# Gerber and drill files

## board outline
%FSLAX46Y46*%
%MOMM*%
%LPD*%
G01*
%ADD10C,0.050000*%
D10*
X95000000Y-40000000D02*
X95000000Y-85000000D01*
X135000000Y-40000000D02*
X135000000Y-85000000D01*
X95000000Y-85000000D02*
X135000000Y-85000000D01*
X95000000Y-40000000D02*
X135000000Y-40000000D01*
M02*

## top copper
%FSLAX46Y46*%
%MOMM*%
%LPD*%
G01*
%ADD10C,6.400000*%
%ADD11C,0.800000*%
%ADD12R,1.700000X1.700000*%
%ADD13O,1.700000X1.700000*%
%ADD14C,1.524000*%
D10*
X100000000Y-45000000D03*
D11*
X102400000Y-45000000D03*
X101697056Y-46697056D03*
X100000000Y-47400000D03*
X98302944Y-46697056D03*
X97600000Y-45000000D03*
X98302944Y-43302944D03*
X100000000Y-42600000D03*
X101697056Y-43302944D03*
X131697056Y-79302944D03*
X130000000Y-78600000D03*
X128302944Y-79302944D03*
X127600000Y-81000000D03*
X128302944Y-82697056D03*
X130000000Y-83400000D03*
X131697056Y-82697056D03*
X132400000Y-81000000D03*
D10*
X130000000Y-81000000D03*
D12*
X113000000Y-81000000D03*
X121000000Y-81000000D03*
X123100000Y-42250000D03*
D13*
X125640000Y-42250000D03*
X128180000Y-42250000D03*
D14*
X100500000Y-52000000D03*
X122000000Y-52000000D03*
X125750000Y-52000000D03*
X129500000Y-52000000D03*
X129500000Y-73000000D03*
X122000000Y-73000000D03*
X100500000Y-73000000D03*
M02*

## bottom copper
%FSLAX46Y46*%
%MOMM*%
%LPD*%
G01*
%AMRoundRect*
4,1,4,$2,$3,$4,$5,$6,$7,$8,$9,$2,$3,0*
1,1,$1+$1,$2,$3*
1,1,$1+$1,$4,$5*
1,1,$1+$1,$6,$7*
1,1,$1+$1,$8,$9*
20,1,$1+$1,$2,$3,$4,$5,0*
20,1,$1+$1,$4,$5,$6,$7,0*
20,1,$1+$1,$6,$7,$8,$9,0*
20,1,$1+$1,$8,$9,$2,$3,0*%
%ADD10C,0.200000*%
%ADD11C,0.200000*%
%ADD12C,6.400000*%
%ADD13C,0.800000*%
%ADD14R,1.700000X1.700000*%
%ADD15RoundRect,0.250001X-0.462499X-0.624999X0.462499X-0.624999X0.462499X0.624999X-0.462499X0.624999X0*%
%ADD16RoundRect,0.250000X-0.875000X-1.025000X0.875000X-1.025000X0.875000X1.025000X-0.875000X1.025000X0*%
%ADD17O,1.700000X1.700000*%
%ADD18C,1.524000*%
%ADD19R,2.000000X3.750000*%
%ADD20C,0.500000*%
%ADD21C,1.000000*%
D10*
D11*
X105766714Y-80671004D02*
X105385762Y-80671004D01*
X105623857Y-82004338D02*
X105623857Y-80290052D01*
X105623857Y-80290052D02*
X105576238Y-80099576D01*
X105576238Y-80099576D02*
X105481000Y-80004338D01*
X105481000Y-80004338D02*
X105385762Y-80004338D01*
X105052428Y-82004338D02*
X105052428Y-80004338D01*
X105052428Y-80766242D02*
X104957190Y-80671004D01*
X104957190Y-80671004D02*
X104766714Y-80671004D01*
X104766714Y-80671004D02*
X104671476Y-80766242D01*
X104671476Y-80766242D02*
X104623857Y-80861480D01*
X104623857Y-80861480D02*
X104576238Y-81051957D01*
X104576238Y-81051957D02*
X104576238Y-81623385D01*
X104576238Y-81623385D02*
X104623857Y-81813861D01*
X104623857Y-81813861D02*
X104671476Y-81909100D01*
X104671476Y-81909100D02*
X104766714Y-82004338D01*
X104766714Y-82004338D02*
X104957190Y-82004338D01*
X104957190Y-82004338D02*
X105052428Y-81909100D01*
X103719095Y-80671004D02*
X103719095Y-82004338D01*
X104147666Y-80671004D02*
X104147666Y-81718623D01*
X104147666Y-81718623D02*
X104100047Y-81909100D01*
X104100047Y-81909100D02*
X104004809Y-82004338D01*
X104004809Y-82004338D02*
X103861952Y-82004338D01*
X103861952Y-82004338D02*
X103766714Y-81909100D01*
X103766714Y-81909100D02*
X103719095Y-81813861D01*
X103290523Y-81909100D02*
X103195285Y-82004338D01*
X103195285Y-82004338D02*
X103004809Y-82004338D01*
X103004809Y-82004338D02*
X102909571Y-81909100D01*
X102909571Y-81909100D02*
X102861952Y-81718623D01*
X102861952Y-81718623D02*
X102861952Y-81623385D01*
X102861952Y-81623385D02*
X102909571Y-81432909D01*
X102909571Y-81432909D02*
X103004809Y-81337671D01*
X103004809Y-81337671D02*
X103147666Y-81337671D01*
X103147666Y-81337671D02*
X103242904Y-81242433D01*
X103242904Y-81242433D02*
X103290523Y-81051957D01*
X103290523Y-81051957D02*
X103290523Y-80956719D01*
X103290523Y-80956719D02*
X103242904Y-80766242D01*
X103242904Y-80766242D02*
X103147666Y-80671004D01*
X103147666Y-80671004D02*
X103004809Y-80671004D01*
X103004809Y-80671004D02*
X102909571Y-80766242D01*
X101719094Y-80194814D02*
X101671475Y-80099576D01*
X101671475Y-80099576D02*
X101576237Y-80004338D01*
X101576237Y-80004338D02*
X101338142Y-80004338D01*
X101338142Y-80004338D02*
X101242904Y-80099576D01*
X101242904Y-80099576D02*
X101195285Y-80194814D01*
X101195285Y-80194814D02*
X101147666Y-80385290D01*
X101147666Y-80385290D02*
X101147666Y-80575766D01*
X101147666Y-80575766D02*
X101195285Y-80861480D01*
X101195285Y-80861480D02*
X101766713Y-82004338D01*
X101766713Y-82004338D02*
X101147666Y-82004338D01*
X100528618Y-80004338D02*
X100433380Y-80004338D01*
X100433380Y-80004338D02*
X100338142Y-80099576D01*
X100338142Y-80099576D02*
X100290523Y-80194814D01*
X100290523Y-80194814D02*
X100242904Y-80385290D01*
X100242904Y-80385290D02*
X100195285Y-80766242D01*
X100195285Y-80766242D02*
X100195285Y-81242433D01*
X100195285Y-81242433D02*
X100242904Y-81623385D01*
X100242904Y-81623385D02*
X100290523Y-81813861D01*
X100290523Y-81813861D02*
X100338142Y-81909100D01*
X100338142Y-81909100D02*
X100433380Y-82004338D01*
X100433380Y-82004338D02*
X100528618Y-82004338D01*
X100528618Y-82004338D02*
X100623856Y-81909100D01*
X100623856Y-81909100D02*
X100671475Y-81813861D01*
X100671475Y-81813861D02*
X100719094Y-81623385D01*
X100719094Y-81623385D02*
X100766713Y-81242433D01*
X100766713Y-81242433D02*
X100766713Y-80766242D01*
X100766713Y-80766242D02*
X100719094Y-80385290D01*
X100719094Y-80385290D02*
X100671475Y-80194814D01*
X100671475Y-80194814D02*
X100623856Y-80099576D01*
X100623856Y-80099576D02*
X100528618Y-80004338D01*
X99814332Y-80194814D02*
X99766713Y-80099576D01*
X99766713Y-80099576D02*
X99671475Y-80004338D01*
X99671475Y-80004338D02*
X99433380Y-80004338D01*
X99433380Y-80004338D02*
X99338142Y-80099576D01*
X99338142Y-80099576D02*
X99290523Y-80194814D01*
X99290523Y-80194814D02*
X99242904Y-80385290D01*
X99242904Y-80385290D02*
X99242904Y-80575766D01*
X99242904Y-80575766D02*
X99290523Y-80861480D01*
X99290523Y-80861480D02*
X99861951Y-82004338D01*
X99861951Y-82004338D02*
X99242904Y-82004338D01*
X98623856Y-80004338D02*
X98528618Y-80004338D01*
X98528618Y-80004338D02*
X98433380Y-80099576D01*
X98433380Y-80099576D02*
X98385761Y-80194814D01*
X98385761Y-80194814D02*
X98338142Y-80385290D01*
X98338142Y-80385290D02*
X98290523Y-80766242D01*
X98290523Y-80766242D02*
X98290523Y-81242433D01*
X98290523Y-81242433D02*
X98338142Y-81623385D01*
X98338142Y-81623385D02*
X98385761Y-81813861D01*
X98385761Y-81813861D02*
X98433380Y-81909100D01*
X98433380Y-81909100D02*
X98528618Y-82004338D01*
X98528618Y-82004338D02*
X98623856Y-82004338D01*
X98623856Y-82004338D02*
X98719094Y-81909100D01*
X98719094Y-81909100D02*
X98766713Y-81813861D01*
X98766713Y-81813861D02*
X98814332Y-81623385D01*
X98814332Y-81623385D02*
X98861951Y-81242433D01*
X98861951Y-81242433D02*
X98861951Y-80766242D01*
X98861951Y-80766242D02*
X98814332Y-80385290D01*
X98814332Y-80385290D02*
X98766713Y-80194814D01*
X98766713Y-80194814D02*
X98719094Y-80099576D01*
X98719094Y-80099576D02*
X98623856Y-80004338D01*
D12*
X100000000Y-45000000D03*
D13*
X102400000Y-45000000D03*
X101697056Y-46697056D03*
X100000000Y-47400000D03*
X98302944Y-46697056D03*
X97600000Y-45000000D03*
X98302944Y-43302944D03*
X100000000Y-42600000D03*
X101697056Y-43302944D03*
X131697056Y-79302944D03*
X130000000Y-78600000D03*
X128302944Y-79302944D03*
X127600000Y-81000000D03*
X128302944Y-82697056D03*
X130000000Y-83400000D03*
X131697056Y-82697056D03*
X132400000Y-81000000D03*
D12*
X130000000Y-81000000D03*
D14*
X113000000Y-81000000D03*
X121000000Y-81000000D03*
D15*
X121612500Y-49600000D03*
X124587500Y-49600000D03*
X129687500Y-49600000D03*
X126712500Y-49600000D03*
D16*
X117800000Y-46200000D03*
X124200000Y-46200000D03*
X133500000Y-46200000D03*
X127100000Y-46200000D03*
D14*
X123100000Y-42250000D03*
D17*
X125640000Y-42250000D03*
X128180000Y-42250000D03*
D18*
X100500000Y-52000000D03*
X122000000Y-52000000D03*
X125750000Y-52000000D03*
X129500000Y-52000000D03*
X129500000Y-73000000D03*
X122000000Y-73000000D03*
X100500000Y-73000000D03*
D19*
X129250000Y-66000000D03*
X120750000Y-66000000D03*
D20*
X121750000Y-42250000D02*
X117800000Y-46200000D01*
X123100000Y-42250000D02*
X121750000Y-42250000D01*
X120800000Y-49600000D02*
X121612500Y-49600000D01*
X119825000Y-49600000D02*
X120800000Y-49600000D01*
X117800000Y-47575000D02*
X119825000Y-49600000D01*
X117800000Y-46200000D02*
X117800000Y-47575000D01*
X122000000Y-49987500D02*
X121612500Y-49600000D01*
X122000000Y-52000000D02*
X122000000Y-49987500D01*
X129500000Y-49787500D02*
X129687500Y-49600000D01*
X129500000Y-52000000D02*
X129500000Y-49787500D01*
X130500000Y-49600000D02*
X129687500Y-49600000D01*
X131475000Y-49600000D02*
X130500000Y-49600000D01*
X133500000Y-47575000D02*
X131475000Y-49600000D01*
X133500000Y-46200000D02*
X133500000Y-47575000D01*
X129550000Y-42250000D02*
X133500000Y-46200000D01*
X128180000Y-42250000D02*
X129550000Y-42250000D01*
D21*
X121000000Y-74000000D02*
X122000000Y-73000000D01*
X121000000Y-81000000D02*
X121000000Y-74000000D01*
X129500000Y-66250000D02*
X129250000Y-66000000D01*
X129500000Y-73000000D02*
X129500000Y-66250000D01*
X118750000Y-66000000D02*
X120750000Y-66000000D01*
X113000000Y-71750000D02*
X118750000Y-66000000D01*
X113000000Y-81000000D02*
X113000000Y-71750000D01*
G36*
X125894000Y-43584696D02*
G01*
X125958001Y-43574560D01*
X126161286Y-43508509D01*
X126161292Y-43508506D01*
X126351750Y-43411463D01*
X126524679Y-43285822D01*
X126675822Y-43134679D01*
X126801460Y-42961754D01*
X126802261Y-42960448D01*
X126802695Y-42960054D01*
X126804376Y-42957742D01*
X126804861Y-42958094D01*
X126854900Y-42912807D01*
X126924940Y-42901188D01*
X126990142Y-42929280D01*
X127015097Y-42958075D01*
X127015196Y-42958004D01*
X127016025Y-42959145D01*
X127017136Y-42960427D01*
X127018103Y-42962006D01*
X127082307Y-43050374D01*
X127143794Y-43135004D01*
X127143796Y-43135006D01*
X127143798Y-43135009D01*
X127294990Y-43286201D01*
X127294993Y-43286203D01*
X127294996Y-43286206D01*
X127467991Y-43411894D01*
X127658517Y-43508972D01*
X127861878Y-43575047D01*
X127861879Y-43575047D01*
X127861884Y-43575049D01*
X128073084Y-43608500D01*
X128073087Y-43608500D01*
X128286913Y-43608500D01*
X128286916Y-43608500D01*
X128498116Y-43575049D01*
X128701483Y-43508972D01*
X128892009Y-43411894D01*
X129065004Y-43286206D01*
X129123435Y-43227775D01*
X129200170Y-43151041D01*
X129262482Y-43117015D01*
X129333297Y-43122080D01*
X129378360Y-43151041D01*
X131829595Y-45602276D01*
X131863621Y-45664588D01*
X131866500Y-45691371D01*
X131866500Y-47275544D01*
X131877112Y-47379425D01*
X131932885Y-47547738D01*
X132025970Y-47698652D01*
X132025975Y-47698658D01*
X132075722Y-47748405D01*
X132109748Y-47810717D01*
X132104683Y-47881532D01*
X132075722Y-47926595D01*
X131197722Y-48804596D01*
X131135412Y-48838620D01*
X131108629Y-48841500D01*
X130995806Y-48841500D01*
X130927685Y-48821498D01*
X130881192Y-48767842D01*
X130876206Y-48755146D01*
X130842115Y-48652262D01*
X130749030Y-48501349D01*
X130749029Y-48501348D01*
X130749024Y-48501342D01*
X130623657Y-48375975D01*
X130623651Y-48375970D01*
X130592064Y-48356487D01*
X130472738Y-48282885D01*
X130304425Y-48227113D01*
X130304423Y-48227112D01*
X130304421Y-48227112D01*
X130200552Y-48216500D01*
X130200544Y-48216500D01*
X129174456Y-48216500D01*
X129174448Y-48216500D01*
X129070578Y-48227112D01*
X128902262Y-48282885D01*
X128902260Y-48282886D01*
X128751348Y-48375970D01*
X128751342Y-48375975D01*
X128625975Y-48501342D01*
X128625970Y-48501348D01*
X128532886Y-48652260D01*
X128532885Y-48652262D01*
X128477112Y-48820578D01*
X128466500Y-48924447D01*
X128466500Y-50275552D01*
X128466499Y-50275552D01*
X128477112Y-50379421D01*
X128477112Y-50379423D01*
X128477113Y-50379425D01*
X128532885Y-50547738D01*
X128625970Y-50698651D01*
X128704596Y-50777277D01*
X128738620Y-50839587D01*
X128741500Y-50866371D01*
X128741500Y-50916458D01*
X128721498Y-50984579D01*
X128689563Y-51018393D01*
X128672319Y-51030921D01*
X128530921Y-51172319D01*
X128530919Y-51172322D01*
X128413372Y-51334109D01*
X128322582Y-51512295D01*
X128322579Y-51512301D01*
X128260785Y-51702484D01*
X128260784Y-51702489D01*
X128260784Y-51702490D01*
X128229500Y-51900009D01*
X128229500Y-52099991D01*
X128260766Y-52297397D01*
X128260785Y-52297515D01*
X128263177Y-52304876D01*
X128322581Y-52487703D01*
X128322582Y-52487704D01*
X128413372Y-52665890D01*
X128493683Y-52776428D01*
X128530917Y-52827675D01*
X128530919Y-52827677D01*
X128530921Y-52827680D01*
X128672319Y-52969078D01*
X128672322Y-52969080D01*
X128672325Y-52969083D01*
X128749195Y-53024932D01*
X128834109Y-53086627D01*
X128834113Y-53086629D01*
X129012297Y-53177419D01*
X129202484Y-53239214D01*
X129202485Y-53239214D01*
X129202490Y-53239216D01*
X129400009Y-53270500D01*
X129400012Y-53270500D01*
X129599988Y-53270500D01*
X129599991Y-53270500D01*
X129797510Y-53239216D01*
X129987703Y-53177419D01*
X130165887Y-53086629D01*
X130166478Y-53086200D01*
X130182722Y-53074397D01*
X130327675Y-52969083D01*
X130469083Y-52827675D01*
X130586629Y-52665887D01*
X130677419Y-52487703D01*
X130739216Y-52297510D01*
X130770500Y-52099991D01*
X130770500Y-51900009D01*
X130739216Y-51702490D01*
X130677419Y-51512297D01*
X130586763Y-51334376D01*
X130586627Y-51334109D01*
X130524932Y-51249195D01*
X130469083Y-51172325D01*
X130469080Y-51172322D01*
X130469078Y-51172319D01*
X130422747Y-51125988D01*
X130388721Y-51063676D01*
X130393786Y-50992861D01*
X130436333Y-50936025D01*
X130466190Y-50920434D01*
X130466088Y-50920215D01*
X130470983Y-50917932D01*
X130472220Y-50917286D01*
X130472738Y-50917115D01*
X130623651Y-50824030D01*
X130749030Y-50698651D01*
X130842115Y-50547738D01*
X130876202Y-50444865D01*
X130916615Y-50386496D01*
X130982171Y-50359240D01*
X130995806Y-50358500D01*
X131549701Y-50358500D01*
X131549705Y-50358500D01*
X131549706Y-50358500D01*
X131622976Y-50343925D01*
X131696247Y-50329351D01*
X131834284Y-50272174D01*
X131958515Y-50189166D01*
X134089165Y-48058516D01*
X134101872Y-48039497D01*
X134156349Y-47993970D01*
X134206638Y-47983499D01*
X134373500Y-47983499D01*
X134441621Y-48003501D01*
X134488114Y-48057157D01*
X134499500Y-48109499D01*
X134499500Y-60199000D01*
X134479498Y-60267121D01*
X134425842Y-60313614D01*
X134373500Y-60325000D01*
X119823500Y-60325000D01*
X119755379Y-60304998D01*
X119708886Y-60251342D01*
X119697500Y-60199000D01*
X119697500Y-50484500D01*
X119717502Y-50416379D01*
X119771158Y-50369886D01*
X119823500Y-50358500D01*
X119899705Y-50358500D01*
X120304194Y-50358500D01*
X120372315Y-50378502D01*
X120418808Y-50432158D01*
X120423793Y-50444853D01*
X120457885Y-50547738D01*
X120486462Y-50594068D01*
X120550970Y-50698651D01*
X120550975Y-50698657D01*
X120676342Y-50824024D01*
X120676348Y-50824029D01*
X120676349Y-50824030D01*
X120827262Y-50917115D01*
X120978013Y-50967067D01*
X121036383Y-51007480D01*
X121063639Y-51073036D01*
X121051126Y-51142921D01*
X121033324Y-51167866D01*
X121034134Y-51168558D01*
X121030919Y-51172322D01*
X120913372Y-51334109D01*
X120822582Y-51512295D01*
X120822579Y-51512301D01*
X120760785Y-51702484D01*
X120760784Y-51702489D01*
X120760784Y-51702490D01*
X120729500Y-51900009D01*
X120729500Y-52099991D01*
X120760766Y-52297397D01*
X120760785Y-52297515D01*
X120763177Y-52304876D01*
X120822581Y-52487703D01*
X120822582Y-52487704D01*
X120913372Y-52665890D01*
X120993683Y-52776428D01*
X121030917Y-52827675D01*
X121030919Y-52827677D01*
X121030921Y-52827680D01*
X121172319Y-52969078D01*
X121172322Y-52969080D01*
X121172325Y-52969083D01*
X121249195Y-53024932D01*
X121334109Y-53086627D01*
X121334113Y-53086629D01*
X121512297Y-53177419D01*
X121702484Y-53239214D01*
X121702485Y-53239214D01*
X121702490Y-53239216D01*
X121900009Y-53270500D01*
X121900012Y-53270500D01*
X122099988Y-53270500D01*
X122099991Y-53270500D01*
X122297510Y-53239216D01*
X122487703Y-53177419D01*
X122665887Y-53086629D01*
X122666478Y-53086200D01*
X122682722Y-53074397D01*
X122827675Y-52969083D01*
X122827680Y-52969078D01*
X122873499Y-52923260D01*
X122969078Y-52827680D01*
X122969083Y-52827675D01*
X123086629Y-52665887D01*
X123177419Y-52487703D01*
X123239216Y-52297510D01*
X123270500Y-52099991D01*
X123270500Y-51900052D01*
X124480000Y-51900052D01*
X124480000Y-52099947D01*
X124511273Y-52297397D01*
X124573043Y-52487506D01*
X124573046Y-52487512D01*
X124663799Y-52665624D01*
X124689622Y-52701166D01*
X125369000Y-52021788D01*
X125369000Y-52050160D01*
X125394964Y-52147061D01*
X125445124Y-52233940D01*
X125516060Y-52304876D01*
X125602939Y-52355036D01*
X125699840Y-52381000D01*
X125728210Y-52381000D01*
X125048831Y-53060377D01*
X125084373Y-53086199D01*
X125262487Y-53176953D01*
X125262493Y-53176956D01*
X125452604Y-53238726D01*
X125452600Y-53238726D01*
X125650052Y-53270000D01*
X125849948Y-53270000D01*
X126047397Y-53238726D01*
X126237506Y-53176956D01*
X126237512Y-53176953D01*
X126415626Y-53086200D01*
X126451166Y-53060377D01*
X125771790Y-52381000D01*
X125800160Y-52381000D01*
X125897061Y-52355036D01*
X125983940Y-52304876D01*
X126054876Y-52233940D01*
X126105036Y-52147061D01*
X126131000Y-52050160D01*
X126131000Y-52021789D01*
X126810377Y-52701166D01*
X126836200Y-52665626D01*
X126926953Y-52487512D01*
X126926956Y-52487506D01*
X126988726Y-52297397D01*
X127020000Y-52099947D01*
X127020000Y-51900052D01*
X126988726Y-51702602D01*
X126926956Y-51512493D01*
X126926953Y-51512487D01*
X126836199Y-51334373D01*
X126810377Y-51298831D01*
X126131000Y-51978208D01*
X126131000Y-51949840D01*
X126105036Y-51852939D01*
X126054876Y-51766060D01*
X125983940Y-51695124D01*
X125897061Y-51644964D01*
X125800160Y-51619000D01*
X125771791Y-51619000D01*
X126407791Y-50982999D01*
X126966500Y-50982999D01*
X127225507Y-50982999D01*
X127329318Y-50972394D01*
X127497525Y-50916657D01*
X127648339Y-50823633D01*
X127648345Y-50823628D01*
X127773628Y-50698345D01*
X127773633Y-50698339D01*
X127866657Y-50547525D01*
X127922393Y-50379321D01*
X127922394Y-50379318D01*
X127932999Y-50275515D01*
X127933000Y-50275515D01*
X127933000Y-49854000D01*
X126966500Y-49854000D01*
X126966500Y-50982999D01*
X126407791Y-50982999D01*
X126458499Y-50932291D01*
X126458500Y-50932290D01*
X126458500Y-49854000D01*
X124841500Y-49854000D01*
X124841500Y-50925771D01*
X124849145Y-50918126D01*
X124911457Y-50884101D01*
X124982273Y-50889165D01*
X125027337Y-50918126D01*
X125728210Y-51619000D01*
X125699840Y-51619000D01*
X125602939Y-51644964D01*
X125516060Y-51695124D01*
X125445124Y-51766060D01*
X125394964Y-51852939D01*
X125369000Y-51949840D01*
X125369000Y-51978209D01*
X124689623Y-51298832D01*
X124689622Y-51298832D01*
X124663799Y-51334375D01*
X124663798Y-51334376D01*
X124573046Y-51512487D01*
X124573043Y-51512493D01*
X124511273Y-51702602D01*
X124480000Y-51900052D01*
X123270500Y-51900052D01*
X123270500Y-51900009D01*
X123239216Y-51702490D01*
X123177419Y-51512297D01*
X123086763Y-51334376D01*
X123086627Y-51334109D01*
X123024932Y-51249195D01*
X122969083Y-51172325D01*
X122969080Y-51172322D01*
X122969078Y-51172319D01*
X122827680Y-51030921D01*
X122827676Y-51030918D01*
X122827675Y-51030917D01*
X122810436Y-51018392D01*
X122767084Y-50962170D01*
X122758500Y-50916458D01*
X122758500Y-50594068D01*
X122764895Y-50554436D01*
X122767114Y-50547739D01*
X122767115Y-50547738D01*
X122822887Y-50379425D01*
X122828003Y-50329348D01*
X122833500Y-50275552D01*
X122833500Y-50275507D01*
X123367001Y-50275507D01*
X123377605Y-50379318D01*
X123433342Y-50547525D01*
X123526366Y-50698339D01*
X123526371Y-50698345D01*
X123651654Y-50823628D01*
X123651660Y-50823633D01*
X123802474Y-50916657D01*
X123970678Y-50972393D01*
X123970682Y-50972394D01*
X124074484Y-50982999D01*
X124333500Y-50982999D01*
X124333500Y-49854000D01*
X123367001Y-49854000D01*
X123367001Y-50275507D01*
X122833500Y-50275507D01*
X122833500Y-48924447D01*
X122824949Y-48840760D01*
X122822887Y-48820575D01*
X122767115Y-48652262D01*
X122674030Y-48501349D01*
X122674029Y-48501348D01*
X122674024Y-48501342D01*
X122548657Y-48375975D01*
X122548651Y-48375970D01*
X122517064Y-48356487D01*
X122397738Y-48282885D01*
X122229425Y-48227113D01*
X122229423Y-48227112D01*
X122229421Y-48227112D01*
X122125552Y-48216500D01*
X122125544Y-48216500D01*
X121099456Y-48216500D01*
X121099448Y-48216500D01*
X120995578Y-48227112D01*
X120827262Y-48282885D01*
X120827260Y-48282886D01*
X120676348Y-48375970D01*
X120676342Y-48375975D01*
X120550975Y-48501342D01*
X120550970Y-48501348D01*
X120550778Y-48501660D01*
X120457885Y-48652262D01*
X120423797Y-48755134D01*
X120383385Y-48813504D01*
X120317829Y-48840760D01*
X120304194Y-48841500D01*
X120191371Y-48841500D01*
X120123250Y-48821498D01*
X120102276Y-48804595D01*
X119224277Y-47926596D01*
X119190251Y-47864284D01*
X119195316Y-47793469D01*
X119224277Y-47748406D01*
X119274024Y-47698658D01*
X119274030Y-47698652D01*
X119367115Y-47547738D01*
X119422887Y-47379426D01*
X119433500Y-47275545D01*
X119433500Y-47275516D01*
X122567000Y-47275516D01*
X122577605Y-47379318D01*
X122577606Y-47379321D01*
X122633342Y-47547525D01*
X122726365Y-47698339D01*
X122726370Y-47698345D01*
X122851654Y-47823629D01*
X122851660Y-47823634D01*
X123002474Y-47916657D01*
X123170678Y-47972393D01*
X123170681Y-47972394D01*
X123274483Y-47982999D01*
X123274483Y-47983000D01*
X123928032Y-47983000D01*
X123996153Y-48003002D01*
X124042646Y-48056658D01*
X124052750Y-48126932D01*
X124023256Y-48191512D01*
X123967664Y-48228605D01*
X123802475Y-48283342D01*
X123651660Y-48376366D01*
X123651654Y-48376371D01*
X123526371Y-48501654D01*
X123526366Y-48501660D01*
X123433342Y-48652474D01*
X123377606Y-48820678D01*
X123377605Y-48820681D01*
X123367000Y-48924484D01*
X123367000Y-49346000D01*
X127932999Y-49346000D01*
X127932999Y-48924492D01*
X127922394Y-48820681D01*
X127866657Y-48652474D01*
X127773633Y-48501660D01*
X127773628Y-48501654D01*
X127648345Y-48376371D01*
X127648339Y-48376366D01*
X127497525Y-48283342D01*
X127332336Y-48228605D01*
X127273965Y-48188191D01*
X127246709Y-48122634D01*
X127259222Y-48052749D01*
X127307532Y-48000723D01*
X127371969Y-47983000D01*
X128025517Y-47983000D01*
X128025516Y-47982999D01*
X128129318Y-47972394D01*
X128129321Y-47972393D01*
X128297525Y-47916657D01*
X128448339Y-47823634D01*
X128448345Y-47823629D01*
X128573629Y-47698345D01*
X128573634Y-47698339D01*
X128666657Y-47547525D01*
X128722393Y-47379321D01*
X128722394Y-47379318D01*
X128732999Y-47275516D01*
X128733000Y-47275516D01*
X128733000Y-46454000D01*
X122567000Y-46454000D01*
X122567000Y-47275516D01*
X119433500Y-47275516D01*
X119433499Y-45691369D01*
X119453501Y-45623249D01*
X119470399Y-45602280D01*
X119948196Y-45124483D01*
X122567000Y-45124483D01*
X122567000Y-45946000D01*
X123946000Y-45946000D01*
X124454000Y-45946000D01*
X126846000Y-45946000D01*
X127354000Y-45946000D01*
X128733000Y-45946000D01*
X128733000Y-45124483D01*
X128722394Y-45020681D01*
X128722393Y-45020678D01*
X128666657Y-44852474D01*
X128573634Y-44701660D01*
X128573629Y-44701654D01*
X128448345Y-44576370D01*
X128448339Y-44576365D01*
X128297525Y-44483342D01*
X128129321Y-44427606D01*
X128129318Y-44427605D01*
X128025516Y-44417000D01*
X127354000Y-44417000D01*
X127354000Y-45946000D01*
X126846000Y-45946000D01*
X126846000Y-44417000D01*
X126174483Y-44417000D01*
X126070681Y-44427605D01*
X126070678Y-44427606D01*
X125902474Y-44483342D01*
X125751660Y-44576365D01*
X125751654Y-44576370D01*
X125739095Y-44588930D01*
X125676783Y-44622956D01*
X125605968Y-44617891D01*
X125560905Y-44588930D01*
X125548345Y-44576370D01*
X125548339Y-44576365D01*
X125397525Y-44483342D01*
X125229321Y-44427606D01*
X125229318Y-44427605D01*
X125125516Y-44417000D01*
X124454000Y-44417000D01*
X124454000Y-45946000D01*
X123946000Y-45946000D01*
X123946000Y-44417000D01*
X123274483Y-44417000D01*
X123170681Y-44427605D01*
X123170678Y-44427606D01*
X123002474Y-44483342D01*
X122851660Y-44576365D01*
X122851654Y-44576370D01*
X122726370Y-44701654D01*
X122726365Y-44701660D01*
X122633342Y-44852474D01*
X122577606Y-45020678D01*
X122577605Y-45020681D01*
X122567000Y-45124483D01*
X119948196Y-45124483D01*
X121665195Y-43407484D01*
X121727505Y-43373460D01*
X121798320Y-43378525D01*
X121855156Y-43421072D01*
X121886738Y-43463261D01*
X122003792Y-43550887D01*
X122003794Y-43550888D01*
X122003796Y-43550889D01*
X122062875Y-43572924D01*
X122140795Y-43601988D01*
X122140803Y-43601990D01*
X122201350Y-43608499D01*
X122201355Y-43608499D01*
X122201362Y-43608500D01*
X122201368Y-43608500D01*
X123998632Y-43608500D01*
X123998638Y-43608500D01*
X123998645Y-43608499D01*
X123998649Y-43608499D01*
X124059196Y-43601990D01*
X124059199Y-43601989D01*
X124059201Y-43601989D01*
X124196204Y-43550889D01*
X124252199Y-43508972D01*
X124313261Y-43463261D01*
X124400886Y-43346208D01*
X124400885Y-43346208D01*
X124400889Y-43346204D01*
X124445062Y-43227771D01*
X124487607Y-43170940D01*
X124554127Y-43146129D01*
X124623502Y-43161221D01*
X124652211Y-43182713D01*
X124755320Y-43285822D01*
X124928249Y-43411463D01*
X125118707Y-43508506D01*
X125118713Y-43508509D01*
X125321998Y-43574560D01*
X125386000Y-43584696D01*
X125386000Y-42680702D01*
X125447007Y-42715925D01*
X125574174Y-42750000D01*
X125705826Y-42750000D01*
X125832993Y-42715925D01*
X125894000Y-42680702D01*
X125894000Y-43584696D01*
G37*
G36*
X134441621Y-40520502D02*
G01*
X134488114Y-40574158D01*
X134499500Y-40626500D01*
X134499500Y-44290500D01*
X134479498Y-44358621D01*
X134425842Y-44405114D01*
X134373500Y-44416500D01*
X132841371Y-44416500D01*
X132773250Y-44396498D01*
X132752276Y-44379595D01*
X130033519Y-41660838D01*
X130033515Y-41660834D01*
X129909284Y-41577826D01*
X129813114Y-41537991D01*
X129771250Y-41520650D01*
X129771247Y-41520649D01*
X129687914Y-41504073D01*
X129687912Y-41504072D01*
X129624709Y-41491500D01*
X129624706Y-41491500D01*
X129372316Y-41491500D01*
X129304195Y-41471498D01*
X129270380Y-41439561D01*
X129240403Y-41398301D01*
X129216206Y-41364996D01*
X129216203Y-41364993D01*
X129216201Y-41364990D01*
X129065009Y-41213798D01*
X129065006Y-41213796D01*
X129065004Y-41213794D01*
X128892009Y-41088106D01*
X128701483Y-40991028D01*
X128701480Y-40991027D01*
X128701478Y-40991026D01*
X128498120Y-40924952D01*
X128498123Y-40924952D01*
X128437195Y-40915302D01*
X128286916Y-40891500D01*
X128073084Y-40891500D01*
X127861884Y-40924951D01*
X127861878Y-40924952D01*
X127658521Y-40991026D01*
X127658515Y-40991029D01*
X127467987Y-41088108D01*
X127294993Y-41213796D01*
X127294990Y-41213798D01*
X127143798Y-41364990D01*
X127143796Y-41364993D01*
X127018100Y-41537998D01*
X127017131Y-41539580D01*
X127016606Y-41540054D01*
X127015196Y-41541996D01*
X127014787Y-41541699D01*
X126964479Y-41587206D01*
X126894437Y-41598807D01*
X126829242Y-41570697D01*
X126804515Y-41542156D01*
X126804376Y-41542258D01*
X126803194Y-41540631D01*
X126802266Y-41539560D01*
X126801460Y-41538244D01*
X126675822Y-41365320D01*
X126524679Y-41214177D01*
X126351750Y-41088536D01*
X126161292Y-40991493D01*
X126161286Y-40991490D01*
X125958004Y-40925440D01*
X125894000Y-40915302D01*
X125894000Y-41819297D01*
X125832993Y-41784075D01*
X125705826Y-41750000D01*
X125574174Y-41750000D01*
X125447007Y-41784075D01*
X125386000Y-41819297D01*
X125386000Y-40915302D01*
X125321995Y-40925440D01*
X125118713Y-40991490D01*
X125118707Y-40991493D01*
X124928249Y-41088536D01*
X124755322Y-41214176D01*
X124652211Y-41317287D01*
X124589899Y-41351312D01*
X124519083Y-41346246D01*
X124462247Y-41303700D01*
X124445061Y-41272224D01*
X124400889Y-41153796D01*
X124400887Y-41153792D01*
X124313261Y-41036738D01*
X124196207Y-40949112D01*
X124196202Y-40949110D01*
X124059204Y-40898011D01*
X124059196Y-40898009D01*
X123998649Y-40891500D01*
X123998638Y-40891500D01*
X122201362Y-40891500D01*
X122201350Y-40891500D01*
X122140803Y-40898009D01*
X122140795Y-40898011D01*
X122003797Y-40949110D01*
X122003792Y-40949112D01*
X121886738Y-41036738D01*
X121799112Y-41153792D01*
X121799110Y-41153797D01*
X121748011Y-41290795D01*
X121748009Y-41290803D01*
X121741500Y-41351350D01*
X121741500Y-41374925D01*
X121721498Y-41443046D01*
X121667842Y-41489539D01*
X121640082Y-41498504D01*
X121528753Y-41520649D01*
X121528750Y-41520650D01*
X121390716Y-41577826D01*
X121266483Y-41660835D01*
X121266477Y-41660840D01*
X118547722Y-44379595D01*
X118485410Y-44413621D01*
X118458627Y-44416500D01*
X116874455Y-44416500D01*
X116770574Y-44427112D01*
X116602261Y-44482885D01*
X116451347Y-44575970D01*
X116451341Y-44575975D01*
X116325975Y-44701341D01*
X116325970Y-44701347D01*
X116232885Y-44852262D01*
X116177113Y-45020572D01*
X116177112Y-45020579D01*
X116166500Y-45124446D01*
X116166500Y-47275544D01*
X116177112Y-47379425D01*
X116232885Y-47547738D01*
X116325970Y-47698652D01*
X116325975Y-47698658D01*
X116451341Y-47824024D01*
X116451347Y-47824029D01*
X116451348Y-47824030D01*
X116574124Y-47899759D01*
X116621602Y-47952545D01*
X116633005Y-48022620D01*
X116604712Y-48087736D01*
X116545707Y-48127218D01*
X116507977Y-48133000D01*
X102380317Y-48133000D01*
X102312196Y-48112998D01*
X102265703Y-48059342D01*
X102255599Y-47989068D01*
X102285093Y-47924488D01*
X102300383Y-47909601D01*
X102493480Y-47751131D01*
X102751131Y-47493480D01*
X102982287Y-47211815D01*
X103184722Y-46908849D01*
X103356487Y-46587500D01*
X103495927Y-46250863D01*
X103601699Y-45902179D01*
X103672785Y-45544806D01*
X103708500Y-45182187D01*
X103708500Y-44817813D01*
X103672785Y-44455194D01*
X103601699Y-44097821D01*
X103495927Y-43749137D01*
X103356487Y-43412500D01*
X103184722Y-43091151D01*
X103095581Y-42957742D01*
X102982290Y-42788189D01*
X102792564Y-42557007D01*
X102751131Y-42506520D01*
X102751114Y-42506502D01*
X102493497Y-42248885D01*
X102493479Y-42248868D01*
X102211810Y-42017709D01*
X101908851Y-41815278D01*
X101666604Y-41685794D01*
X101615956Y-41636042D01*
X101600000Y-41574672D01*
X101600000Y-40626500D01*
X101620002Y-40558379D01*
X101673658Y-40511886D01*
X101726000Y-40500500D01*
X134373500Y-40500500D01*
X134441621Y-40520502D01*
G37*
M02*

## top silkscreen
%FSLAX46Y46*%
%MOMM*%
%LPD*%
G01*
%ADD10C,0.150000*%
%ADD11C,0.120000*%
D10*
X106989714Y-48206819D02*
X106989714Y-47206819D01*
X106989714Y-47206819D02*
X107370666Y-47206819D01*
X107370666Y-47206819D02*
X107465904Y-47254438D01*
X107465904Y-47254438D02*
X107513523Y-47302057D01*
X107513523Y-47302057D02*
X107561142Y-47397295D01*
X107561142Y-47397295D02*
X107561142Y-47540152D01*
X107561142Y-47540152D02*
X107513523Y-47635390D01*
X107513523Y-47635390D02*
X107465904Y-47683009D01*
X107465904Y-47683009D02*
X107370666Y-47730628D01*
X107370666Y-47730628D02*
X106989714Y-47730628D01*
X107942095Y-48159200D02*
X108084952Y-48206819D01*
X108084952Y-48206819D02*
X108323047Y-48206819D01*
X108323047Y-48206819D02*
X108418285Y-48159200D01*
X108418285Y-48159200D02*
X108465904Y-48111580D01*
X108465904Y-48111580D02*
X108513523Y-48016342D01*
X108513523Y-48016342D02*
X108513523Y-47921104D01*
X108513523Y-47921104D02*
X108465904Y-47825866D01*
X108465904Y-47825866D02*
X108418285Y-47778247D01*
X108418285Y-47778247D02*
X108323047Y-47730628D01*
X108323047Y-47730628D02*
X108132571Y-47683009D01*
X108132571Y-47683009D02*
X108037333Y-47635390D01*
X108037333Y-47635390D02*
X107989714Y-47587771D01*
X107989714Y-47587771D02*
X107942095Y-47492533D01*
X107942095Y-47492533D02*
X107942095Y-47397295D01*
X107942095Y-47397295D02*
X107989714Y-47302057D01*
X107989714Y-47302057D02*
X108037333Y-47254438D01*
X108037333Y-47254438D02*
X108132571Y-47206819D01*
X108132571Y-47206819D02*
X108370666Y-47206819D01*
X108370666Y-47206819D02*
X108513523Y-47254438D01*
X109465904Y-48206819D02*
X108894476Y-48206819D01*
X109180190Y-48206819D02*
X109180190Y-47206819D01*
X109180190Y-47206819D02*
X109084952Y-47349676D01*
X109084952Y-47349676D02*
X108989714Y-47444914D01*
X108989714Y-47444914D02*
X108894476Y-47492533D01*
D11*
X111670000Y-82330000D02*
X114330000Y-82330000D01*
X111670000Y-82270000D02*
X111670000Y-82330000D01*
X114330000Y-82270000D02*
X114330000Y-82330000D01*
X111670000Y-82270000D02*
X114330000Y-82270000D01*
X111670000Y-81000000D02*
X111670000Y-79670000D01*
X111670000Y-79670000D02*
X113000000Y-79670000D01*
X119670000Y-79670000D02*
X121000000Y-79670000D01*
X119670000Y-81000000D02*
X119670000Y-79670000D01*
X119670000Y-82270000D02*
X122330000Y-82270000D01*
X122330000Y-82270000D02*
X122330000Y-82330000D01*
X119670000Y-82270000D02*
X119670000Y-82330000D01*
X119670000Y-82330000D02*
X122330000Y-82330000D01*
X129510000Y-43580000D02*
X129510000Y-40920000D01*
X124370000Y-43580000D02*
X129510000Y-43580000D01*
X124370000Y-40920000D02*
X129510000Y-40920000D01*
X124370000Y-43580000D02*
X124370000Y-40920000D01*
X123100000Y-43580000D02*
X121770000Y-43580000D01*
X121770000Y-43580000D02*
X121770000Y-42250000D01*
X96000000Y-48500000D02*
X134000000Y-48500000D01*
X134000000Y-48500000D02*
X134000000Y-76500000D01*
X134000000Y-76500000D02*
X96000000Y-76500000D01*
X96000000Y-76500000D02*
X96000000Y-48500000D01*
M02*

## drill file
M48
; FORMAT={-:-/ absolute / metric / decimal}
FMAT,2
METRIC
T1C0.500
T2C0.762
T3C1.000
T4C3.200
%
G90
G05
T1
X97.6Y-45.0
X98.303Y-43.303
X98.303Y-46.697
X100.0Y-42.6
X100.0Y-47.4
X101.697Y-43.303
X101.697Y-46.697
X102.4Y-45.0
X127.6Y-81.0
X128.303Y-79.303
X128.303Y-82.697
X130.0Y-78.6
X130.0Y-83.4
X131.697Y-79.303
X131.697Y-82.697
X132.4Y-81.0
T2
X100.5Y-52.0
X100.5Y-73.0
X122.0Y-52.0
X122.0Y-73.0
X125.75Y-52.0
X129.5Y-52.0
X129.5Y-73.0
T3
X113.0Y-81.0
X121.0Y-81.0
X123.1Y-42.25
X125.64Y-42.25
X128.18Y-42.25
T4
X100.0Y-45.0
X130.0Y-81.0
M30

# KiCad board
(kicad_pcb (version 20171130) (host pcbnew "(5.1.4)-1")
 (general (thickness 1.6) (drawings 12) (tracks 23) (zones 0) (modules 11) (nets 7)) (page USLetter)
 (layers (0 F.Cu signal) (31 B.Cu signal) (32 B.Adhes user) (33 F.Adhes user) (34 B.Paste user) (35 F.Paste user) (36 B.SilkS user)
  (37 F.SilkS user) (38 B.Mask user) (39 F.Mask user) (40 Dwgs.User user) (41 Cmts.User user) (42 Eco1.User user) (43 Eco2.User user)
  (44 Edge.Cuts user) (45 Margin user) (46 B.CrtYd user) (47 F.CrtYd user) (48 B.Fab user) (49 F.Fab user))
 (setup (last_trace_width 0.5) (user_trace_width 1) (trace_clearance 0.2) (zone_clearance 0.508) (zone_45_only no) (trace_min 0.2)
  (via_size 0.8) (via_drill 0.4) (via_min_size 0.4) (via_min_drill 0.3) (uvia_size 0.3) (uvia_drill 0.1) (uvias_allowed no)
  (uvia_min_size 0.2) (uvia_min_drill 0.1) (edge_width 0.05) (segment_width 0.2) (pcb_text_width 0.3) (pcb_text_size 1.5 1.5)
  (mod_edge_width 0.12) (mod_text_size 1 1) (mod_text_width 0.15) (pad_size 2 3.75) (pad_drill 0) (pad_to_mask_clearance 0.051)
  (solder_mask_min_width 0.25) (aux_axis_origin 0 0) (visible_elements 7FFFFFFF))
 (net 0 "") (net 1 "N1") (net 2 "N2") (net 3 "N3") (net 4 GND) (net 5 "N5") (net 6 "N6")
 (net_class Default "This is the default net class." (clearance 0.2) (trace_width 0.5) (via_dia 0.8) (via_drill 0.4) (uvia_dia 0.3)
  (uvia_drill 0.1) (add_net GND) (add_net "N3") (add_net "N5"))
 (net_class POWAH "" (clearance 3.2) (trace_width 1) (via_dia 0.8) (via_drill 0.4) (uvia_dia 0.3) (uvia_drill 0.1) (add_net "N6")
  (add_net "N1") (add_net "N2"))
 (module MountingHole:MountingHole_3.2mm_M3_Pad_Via (layer F.Cu) (at 100 45)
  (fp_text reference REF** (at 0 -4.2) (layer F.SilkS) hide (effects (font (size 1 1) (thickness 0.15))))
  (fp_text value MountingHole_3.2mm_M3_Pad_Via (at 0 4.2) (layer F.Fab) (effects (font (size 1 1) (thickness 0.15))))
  (pad 1 thru_hole circle (at 0 0) (size 6.4 6.4) (drill 3.2) (layers *.Cu *.Mask))
  (pad 1 thru_hole circle (at 2.4 0) (size 0.8 0.8) (drill 0.5) (layers *.Cu *.Mask))
  (pad 1 thru_hole circle (at 1.697056 1.697056) (size 0.8 0.8) (drill 0.5) (layers *.Cu *.Mask))
  (pad 1 thru_hole circle (at 0 2.4) (size 0.8 0.8) (drill 0.5) (layers *.Cu *.Mask))
  (pad 1 thru_hole circle (at -1.697056 1.697056) (size 0.8 0.8) (drill 0.5) (layers *.Cu *.Mask))
  (pad 1 thru_hole circle (at -2.4 0) (size 0.8 0.8) (drill 0.5) (layers *.Cu *.Mask))
  (pad 1 thru_hole circle (at -1.697056 -1.697056) (size 0.8 0.8) (drill 0.5) (layers *.Cu *.Mask))
  (pad 1 thru_hole circle (at 0 -2.4) (size 0.8 0.8) (drill 0.5) (layers *.Cu *.Mask))
  (pad 1 thru_hole circle (at 1.697056 -1.697056) (size 0.8 0.8) (drill 0.5) (layers *.Cu *.Mask)))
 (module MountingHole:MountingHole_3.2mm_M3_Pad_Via (layer F.Cu) (at 130 81)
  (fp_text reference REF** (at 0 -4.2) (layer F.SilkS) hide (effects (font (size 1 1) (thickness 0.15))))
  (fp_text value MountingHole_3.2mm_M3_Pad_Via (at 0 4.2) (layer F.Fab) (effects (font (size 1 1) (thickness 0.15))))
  (pad 1 thru_hole circle (at 1.697056 -1.697056) (size 0.8 0.8) (drill 0.5) (layers *.Cu *.Mask))
  (pad 1 thru_hole circle (at 0 -2.4) (size 0.8 0.8) (drill 0.5) (layers *.Cu *.Mask))
  (pad 1 thru_hole circle (at -1.697056 -1.697056) (size 0.8 0.8) (drill 0.5) (layers *.Cu *.Mask))
  (pad 1 thru_hole circle (at -2.4 0) (size 0.8 0.8) (drill 0.5) (layers *.Cu *.Mask))
  (pad 1 thru_hole circle (at -1.697056 1.697056) (size 0.8 0.8) (drill 0.5) (layers *.Cu *.Mask))
  (pad 1 thru_hole circle (at 0 2.4) (size 0.8 0.8) (drill 0.5) (layers *.Cu *.Mask))
  (pad 1 thru_hole circle (at 1.697056 1.697056) (size 0.8 0.8) (drill 0.5) (layers *.Cu *.Mask))
  (pad 1 thru_hole circle (at 2.4 0) (size 0.8 0.8) (drill 0.5) (layers *.Cu *.Mask))
  (pad 1 thru_hole circle (at 0 0) (size 6.4 6.4) (drill 3.2) (layers *.Cu *.Mask)))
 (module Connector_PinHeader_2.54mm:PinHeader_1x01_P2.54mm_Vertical (layer F.Cu) (at 113 81)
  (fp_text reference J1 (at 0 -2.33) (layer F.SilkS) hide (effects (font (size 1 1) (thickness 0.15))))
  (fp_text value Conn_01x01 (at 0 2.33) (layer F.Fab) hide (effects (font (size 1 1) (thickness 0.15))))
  (fp_line (start -1.33 1.33) (end 1.33 1.33) (layer F.SilkS) (width 0.12))
  (fp_line (start -1.33 1.27) (end -1.33 1.33) (layer F.SilkS) (width 0.12))
  (fp_line (start 1.33 1.27) (end 1.33 1.33) (layer F.SilkS) (width 0.12))
  (fp_line (start -1.33 1.27) (end 1.33 1.27) (layer F.SilkS) (width 0.12))
  (fp_line (start -1.33 0) (end -1.33 -1.33) (layer F.SilkS) (width 0.12))
  (fp_line (start -1.33 -1.33) (end 0 -1.33) (layer F.SilkS) (width 0.12))
  (pad 1 thru_hole rect (at 0 0) (size 1.7 1.7) (drill 1) (layers *.Cu *.Mask) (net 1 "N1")))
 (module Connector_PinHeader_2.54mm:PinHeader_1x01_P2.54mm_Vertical (layer F.Cu) (at 121 81)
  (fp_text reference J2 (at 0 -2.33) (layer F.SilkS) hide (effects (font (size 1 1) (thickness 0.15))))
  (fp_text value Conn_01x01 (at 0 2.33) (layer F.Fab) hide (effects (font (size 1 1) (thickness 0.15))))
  (fp_line (start -1.33 -1.33) (end 0 -1.33) (layer F.SilkS) (width 0.12))
  (fp_line (start -1.33 0) (end -1.33 -1.33) (layer F.SilkS) (width 0.12))
  (fp_line (start -1.33 1.27) (end 1.33 1.27) (layer F.SilkS) (width 0.12))
  (fp_line (start 1.33 1.27) (end 1.33 1.33) (layer F.SilkS) (width 0.12))
  (fp_line (start -1.33 1.27) (end -1.33 1.33) (layer F.SilkS) (width 0.12))
  (fp_line (start -1.33 1.33) (end 1.33 1.33) (layer F.SilkS) (width 0.12))
  (pad 1 thru_hole rect (at 0 0) (size 1.7 1.7) (drill 1) (layers *.Cu *.Mask) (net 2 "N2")))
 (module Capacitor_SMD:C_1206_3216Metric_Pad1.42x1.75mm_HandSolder (layer B.Cu) (at 123.1 49.6)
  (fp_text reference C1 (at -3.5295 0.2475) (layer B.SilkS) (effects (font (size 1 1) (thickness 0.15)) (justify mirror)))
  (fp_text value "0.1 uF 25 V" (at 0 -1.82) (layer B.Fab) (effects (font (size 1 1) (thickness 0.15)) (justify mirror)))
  (pad 1 smd roundrect (at -1.4875 0) (size 1.425 1.75) (layers B.Cu B.Paste B.Mask) (roundrect_rratio 0.175439) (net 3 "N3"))
  (pad 2 smd roundrect (at 1.4875 0) (size 1.425 1.75) (layers B.Cu B.Paste B.Mask) (roundrect_rratio 0.175439) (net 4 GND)))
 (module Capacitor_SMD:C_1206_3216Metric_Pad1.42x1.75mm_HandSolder (layer B.Cu) (at 128.2 49.6)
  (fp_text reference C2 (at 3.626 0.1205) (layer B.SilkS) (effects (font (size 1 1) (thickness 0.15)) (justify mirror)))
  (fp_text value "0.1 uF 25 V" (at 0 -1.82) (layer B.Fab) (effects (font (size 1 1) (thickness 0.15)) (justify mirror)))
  (pad 2 smd roundrect (at 1.4875 0) (size 1.425 1.75) (layers B.Cu B.Paste B.Mask) (roundrect_rratio 0.175439) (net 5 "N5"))
  (pad 1 smd roundrect (at -1.4875 0) (size 1.425 1.75) (layers B.Cu B.Paste B.Mask) (roundrect_rratio 0.175439) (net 4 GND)))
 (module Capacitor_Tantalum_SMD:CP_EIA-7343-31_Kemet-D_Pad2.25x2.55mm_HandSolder (layer B.Cu) (at 121 46.2)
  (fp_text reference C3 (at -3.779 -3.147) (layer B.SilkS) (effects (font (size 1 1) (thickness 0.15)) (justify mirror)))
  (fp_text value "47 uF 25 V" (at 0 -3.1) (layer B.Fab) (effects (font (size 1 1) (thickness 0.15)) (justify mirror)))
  (pad 1 smd roundrect (at -3.2 0) (size 2.25 2.55) (layers B.Cu B.Paste B.Mask) (roundrect_rratio 0.111111) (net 3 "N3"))
  (pad 2 smd roundrect (at 3.2 0) (size 2.25 2.55) (layers B.Cu B.Paste B.Mask) (roundrect_rratio 0.111111) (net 4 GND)))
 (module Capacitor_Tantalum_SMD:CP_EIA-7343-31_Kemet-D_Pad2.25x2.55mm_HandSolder (layer B.Cu) (at 130.3 46.2)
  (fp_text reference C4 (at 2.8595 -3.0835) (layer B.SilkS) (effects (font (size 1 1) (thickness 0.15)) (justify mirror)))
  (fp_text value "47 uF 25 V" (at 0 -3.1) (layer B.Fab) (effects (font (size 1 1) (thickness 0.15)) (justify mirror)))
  (pad 2 smd roundrect (at 3.2 0) (size 2.25 2.55) (layers B.Cu B.Paste B.Mask) (roundrect_rratio 0.111111) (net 5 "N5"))
  (pad 1 smd roundrect (at -3.2 0) (size 2.25 2.55) (layers B.Cu B.Paste B.Mask) (roundrect_rratio 0.111111) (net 4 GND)))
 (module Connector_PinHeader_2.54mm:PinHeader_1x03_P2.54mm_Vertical (layer F.Cu) (at 123.1 42.25 90)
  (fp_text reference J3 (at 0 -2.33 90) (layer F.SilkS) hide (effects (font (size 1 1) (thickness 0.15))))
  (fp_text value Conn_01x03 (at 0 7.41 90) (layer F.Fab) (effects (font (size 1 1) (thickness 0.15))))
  (fp_line (start -1.33 6.41) (end 1.33 6.41) (layer F.SilkS) (width 0.12))
  (fp_line (start -1.33 1.27) (end -1.33 6.41) (layer F.SilkS) (width 0.12))
  (fp_line (start 1.33 1.27) (end 1.33 6.41) (layer F.SilkS) (width 0.12))
  (fp_line (start -1.33 1.27) (end 1.33 1.27) (layer F.SilkS) (width 0.12))
  (fp_line (start -1.33 0) (end -1.33 -1.33) (layer F.SilkS) (width 0.12))
  (fp_line (start -1.33 -1.33) (end 0 -1.33) (layer F.SilkS) (width 0.12))
  (pad 1 thru_hole rect (at 0 0 90) (size 1.7 1.7) (drill 1) (layers *.Cu *.Mask) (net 3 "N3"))
  (pad 2 thru_hole oval (at 0 2.54 90) (size 1.7 1.7) (drill 1) (layers *.Cu *.Mask) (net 4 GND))
  (pad 3 thru_hole oval (at 0 5.08 90) (size 1.7 1.7) (drill 1) (layers *.Cu *.Mask) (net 5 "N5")))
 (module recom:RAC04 (layer F.Cu) (at 115 62.5)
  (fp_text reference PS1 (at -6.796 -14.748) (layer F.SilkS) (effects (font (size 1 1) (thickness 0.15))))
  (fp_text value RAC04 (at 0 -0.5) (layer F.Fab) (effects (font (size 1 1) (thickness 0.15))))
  (fp_line (start -19 -14) (end 19 -14) (layer F.SilkS) (width 0.12))
  (fp_line (start 19 -14) (end 19 14) (layer F.SilkS) (width 0.12))
  (fp_line (start 19 14) (end -19 14) (layer F.SilkS) (width 0.12))
  (fp_line (start -19 14) (end -19 -14) (layer F.SilkS) (width 0.12))
  (pad 1 thru_hole circle (at -14.5 -10.5) (size 1.524 1.524) (drill 0.762) (layers *.Cu *.Mask))
  (pad 2 thru_hole circle (at 7 -10.5) (size 1.524 1.524) (drill 0.762) (layers *.Cu *.Mask) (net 3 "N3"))
  (pad 3 thru_hole circle (at 10.75 -10.5) (size 1.524 1.524) (drill 0.762) (layers *.Cu *.Mask) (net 4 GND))
  (pad 4 thru_hole circle (at 14.5 -10.5) (size 1.524 1.524) (drill 0.762) (layers *.Cu *.Mask) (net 5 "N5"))
  (pad 5 thru_hole circle (at 14.5 10.5) (size 1.524 1.524) (drill 0.762) (layers *.Cu *.Mask) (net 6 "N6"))
  (pad 6 thru_hole circle (at 7 10.5) (size 1.524 1.524) (drill 0.762) (layers *.Cu *.Mask) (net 2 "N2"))
  (pad 7 thru_hole circle (at -14.5 10.5) (size 1.524 1.524) (drill 0.762) (layers *.Cu *.Mask)))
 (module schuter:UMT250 (layer B.Cu) (at 125 66 180)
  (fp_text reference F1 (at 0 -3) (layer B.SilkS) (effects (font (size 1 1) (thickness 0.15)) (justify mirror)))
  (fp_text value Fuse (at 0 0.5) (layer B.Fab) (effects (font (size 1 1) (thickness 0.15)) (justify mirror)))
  (pad 1 smd rect (at -4.25 0 180) (size 2 3.75) (layers B.Cu B.Paste B.Mask) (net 6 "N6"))
  (pad 2 smd rect (at 4.25 0 180) (size 2 3.75) (layers B.Cu B.Paste B.Mask) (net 1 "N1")))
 (gr_line (start 95 40) (end 95 85) (layer Edge.Cuts) (width 0.05))
 (gr_line (start 135 40) (end 135 85) (layer Edge.Cuts) (width 0.05))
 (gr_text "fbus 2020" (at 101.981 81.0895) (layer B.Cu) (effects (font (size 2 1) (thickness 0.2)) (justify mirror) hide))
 (gr_line (start 95 85) (end 135 85) (layer Edge.Cuts) (width 0.05))
 (gr_line (start 95 40) (end 135 40) (layer Edge.Cuts) (width 0.05))
 (segment (start 121.75 42.25) (end 117.8 46.2) (width 0.5) (layer B.Cu) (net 3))
 (segment (start 123.1 42.25) (end 121.75 42.25) (width 0.5) (layer B.Cu) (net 3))
 (segment (start 120.8 49.6) (end 121.6125 49.6) (width 0.5) (layer B.Cu) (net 3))
 (segment (start 119.825 49.6) (end 120.8 49.6) (width 0.5) (layer B.Cu) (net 3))
 (segment (start 117.8 47.575) (end 119.825 49.6) (width 0.5) (layer B.Cu) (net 3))
 (segment (start 117.8 46.2) (end 117.8 47.575) (width 0.5) (layer B.Cu) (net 3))
 (segment (start 122 49.9875) (end 121.6125 49.6) (width 0.5) (layer B.Cu) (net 3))
 (segment (start 122 52) (end 122 49.9875) (width 0.5) (layer B.Cu) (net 3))
 (segment (start 129.5 49.7875) (end 129.6875 49.6) (width 0.5) (layer B.Cu) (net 5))
 (segment (start 129.5 52) (end 129.5 49.7875) (width 0.5) (layer B.Cu) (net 5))
 (segment (start 130.5 49.6) (end 129.6875 49.6) (width 0.5) (layer B.Cu) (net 5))
 (segment (start 131.475 49.6) (end 130.5 49.6) (width 0.5) (layer B.Cu) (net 5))
 (segment (start 133.5 47.575) (end 131.475 49.6) (width 0.5) (layer B.Cu) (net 5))
 (segment (start 133.5 46.2) (end 133.5 47.575) (width 0.5) (layer B.Cu) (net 5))
 (segment (start 129.55 42.25) (end 133.5 46.2) (width 0.5) (layer B.Cu) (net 5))
 (segment (start 128.18 42.25) (end 129.55 42.25) (width 0.5) (layer B.Cu) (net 5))
 (segment (start 121 74) (end 122 73) (width 1) (layer B.Cu) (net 2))
 (segment (start 121 81) (end 121 74) (width 1) (layer B.Cu) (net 2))
 (segment (start 129.5 66.25) (end 129.25 66) (width 1) (layer B.Cu) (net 6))
 (segment (start 129.5 73) (end 129.5 66.25) (width 1) (layer B.Cu) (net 6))
 (segment (start 118.75 66) (end 120.75 66) (width 1) (layer B.Cu) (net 1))
 (segment (start 113 71.75) (end 118.75 66) (width 1) (layer B.Cu) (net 1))
 (segment (start 113 81) (end 113 71.75) (width 1) (layer B.Cu) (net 1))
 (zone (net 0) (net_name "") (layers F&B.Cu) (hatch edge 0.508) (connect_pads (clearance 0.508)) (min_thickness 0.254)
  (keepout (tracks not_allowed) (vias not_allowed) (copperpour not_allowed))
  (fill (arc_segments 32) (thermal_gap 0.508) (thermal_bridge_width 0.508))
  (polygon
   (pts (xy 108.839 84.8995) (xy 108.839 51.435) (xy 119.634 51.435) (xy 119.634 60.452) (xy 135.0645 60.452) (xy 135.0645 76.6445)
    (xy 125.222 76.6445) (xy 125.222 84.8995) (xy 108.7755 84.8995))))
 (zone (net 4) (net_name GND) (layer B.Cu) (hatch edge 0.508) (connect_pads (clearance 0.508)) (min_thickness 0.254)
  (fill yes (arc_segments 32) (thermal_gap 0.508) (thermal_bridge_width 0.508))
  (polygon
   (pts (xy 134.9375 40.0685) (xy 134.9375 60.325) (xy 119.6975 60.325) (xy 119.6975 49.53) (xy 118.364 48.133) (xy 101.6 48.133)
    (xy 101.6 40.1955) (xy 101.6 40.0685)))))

